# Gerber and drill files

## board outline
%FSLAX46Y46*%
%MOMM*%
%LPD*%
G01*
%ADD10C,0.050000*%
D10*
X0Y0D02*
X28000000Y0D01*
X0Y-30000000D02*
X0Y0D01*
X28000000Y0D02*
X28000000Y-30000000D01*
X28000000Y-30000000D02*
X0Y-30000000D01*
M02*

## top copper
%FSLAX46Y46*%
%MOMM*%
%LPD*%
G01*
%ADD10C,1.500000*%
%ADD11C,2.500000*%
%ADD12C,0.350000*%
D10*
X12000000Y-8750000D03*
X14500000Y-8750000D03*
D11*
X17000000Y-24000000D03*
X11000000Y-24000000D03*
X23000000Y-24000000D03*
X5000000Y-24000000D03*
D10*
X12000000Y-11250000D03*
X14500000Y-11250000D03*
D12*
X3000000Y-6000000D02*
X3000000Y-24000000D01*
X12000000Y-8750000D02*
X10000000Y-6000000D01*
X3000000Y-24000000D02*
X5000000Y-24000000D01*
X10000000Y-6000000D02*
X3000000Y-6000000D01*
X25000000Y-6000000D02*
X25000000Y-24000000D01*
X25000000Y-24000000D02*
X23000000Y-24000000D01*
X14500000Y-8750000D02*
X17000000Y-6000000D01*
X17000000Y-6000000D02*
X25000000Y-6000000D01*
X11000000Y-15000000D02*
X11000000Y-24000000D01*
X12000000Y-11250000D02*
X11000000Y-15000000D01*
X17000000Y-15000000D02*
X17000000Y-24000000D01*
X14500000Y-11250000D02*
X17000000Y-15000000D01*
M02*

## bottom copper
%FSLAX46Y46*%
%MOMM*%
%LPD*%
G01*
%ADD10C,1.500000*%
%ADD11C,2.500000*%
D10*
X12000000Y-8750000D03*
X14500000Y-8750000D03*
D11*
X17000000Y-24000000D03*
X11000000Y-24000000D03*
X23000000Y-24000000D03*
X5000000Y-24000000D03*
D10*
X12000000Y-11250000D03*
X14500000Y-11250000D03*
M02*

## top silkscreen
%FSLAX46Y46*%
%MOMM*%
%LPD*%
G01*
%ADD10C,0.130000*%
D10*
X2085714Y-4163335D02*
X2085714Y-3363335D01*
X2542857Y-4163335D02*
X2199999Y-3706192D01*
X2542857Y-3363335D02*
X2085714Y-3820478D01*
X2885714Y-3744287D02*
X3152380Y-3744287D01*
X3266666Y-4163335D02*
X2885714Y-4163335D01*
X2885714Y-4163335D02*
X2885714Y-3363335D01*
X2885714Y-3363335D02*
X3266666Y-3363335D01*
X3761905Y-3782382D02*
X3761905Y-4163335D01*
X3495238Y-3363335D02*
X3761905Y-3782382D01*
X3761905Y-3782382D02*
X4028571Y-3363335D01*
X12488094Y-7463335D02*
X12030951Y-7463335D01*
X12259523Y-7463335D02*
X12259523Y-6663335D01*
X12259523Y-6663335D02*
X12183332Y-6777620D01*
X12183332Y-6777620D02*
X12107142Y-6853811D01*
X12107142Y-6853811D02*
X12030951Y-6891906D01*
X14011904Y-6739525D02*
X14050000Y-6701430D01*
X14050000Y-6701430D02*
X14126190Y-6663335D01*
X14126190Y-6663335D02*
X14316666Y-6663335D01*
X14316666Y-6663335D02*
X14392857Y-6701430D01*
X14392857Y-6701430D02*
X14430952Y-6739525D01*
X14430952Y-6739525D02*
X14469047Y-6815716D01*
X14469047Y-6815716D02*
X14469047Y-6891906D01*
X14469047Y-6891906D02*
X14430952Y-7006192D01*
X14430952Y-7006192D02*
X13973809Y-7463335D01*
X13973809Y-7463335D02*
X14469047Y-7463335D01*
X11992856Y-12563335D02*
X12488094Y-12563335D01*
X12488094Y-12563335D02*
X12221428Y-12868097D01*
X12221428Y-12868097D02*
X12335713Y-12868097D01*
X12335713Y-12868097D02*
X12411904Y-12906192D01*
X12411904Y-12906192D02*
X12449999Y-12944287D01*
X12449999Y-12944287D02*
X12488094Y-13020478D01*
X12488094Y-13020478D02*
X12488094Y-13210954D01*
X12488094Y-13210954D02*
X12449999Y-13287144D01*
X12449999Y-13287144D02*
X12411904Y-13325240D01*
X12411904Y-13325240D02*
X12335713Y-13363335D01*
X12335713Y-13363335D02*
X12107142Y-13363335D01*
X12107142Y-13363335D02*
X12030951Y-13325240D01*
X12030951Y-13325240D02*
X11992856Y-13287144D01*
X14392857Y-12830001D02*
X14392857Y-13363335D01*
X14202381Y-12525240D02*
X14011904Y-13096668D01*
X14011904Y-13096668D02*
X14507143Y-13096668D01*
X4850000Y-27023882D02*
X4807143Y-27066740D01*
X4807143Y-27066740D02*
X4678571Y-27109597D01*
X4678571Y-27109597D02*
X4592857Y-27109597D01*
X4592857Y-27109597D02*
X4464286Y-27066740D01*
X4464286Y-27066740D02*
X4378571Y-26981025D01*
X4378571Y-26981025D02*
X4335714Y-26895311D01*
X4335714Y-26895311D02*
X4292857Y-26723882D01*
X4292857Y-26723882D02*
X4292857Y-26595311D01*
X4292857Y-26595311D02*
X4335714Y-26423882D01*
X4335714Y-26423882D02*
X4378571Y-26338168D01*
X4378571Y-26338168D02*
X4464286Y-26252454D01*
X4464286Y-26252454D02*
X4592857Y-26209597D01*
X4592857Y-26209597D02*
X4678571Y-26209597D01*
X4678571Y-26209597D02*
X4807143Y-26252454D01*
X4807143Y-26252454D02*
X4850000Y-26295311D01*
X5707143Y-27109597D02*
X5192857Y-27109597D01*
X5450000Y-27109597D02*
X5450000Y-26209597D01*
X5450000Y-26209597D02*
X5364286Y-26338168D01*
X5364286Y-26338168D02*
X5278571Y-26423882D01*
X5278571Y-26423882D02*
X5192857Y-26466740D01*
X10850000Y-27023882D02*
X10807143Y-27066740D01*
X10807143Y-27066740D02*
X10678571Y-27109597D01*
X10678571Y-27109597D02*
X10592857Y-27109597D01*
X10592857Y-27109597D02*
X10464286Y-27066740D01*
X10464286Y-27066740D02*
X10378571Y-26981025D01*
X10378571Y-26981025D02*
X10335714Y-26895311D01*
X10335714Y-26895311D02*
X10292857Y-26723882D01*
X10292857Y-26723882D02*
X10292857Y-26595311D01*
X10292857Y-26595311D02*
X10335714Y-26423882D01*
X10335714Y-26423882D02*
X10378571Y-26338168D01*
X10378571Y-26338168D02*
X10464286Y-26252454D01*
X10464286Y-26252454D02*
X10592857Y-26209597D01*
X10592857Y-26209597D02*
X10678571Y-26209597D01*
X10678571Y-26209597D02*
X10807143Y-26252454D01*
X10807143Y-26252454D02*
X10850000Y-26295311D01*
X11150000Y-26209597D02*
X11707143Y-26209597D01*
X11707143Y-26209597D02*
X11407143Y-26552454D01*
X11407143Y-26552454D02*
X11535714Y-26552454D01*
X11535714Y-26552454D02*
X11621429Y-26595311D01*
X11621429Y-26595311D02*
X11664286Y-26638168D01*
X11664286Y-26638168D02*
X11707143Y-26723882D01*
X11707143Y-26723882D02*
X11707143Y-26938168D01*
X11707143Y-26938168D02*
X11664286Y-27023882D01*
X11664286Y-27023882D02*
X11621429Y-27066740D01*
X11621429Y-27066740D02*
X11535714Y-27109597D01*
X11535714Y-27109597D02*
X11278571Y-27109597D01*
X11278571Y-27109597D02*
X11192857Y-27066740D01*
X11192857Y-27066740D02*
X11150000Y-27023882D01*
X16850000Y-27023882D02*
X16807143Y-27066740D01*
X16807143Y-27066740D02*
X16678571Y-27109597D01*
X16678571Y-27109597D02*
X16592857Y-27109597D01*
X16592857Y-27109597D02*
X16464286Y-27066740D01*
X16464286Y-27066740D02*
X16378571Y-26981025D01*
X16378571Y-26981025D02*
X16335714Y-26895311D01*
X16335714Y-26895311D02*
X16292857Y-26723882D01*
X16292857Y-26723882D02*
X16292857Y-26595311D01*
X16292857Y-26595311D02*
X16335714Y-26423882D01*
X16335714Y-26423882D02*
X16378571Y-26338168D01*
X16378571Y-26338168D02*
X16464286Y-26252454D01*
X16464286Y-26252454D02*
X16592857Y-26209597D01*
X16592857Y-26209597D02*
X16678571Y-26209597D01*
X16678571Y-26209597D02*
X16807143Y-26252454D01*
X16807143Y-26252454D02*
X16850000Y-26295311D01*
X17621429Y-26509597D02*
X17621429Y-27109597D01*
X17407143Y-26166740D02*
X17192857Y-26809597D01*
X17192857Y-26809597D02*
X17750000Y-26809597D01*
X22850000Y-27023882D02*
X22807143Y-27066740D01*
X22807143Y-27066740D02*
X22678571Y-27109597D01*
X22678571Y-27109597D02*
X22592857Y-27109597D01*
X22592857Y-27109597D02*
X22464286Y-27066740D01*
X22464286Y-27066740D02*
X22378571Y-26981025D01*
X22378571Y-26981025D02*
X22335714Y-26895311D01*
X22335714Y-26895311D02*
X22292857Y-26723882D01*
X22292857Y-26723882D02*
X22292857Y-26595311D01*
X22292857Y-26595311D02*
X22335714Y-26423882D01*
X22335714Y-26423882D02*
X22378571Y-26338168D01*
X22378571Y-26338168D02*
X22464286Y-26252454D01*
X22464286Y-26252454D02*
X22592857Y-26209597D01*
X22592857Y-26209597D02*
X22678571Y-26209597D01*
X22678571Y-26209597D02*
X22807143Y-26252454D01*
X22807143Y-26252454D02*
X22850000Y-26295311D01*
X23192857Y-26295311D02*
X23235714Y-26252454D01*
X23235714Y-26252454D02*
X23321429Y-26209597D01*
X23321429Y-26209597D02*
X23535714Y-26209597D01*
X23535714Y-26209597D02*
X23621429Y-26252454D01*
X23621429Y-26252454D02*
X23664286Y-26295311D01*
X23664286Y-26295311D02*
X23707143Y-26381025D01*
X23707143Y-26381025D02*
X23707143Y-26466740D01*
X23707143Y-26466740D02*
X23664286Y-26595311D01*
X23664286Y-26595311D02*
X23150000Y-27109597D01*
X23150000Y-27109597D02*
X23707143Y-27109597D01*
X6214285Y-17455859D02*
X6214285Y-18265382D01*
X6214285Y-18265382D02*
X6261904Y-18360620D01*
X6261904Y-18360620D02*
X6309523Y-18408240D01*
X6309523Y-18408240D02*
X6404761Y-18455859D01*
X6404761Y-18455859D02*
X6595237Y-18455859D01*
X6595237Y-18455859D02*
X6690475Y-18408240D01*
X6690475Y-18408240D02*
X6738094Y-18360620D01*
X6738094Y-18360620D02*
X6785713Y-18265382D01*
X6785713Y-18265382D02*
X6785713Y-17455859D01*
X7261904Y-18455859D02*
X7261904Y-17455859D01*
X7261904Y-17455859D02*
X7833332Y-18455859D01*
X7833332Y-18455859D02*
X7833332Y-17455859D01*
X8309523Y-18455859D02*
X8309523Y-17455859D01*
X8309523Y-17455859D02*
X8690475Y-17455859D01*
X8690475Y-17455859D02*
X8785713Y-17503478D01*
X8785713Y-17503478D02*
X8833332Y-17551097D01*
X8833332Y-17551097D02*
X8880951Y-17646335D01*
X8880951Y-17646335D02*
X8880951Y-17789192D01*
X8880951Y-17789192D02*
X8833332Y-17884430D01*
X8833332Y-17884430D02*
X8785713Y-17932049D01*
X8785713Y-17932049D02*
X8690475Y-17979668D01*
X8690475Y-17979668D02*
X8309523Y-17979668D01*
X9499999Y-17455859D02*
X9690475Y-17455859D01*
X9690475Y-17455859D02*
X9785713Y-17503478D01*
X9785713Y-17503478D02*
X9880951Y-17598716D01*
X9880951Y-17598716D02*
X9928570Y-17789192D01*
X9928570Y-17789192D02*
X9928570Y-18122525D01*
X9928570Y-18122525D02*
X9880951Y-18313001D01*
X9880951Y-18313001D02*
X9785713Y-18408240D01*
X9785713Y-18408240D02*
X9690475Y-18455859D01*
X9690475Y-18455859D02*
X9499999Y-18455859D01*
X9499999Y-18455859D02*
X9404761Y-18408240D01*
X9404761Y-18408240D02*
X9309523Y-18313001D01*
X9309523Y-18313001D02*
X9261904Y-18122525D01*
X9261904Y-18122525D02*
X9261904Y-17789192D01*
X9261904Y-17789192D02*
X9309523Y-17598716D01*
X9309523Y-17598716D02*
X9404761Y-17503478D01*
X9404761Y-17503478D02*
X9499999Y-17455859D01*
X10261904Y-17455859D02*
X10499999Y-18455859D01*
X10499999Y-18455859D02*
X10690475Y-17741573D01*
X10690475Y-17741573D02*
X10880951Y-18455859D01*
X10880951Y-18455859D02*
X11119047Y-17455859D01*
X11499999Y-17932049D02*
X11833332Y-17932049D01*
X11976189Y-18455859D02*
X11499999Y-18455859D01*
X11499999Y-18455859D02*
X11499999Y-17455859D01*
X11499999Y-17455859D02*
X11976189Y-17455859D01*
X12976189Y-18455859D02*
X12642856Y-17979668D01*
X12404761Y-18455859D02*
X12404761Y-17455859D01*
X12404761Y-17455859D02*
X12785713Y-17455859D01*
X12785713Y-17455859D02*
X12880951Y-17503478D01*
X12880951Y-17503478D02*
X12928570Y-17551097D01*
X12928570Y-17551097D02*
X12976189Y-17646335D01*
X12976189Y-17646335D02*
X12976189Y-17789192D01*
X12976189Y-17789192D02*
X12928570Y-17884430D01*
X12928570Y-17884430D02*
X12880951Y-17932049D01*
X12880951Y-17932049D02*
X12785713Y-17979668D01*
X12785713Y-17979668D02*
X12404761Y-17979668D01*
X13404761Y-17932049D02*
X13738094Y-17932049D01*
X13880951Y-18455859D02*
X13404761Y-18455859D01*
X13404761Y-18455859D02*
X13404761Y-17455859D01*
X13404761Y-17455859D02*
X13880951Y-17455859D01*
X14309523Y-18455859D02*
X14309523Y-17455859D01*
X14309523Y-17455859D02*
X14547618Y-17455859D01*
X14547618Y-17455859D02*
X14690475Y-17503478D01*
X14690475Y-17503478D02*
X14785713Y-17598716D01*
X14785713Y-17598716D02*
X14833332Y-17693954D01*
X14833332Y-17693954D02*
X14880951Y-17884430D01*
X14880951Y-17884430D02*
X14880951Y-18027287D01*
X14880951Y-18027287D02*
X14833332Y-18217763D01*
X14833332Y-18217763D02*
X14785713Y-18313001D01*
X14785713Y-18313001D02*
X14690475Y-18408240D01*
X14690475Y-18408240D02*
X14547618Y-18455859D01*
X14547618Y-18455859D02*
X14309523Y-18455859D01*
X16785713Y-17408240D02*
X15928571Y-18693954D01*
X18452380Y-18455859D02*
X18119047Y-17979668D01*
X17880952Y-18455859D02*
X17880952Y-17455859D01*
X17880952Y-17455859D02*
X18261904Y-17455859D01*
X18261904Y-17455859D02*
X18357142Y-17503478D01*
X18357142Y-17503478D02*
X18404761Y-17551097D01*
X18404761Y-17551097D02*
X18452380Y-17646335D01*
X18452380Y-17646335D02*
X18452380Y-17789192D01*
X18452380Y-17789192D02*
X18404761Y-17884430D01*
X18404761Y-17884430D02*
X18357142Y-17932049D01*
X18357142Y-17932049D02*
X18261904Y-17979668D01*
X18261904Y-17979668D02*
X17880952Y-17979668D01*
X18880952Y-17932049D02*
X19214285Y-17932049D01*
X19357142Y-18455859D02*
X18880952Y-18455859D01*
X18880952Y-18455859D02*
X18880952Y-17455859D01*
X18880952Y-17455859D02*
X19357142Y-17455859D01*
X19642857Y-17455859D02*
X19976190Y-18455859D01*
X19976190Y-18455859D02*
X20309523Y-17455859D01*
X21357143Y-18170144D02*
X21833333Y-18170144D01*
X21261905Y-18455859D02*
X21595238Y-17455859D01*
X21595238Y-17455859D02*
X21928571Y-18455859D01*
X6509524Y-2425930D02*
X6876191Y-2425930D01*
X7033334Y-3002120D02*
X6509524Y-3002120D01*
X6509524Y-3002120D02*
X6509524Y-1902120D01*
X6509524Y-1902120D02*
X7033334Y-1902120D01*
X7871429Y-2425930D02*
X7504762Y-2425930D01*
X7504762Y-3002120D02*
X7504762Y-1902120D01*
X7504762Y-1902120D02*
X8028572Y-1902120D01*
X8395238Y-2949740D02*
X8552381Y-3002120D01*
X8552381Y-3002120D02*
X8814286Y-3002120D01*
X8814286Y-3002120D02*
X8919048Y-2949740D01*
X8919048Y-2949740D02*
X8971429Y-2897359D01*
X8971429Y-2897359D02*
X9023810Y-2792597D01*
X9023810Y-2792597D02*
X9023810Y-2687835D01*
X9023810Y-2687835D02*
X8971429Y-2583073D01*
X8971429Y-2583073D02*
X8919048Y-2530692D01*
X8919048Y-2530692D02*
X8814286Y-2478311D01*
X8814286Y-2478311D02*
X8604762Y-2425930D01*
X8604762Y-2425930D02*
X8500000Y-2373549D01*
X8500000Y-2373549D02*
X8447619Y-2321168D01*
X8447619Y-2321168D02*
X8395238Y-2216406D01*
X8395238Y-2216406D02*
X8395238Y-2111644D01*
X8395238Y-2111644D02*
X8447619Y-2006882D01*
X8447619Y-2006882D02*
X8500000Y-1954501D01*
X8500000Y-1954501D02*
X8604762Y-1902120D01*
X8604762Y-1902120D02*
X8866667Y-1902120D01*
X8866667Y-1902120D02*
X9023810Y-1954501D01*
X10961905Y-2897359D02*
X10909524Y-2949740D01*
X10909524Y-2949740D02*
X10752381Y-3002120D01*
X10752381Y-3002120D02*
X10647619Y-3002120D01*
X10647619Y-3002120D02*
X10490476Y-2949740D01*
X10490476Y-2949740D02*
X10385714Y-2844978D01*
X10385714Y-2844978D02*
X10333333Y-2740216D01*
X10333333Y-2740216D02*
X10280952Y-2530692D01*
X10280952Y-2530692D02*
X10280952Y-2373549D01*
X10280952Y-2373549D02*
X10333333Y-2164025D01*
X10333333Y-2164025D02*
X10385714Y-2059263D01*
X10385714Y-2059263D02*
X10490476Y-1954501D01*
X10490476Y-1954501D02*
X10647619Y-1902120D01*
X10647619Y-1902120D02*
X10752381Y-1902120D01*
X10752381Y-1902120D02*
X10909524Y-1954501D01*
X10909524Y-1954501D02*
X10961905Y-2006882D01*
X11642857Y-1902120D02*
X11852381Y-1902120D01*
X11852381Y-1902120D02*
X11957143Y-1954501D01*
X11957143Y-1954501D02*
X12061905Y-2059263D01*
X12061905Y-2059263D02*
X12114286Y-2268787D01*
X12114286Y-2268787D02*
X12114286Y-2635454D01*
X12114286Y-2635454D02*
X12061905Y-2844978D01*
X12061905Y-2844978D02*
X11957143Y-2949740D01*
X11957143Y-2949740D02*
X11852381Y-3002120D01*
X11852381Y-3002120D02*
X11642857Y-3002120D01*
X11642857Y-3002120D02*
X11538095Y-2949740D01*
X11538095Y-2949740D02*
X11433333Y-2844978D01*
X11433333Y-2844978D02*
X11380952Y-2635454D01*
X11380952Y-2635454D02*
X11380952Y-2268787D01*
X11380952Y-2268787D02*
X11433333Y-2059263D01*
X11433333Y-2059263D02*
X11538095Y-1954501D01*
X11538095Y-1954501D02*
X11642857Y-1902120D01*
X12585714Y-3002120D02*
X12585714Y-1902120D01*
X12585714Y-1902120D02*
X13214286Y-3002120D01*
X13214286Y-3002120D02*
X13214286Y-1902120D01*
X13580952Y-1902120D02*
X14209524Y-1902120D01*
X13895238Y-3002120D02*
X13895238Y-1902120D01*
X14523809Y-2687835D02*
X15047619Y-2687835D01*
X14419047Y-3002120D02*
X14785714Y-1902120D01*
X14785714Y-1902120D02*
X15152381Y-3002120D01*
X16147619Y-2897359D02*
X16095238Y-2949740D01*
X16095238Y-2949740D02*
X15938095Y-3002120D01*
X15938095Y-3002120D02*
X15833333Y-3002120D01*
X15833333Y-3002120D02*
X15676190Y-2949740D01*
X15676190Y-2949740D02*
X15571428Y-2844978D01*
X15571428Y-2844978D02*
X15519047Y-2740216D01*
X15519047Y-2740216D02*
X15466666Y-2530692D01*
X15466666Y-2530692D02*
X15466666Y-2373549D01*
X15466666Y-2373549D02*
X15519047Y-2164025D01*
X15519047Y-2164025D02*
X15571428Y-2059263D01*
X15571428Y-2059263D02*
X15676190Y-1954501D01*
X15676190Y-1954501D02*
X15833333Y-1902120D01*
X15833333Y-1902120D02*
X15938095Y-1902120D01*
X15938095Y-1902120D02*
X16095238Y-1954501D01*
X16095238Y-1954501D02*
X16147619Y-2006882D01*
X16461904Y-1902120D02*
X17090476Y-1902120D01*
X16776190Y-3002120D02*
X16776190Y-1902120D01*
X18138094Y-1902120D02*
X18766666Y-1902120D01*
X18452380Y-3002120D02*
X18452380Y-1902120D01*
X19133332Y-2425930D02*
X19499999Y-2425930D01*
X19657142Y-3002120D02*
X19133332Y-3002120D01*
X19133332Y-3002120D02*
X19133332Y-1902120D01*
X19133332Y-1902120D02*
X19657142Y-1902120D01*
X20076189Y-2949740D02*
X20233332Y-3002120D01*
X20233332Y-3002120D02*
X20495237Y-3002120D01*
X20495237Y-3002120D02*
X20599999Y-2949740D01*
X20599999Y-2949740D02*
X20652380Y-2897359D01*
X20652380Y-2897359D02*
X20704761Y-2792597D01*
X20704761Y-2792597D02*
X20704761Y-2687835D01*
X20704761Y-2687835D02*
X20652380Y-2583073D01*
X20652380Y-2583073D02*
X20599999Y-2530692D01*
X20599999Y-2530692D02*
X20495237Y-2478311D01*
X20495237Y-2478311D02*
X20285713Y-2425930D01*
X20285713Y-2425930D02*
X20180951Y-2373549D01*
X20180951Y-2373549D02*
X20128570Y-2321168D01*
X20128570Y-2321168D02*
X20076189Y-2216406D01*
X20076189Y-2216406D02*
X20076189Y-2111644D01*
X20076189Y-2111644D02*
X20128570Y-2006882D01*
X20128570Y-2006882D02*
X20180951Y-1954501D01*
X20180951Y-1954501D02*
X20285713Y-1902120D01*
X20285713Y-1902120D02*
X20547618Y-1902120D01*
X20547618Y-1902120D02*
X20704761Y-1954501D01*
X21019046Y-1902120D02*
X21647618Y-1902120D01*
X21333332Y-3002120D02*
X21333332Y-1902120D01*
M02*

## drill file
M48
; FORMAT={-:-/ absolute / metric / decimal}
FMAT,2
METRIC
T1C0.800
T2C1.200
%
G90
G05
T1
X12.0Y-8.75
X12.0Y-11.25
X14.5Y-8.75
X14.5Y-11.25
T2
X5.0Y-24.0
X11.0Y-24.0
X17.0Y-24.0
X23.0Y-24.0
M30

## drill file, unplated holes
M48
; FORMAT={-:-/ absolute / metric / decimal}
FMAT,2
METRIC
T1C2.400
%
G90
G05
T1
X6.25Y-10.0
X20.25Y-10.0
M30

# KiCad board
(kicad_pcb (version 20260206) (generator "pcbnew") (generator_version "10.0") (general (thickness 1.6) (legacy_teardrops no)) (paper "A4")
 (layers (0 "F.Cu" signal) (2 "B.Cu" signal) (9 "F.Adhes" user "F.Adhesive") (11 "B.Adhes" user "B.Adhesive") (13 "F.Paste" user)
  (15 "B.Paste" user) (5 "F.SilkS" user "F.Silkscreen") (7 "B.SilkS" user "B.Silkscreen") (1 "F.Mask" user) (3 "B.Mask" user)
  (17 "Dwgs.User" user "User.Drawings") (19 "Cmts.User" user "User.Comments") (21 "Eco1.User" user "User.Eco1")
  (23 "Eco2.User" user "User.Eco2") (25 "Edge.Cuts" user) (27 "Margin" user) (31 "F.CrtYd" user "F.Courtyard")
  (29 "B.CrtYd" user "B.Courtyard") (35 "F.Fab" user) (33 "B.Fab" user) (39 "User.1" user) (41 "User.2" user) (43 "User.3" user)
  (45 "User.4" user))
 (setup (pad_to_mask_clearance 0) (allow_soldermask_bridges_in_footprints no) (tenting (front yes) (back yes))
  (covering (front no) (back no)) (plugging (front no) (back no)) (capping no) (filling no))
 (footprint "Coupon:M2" (layer "F.Cu") (at 6.25 10)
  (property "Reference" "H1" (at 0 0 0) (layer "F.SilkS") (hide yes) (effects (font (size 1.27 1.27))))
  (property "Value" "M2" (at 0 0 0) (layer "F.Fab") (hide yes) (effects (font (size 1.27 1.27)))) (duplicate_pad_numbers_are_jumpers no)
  (pad "" np_thru_hole circle (at 0 0) (size 2.4 2.4) (drill 2.4) (layers "*.Cu" "*.Mask")))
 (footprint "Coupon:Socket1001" (layer "F.Cu") (at 12 8.75)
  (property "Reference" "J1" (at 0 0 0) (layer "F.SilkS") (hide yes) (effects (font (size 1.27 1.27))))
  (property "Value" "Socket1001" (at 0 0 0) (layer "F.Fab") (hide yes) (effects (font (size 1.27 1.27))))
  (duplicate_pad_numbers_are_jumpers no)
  (pad "1" thru_hole circle (at 0 0) (size 1.5 1.5) (drill 0.8) (layers "*.Cu" "*.Mask") (remove_unused_layers no) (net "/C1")))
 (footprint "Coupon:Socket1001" (layer "F.Cu") (at 14.5 8.75)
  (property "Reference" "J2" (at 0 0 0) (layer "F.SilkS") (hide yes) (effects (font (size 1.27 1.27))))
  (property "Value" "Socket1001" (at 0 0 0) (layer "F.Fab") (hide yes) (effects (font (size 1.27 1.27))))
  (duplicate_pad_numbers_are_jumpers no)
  (pad "1" thru_hole circle (at 0 0) (size 1.5 1.5) (drill 0.8) (layers "*.Cu" "*.Mask") (remove_unused_layers no) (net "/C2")))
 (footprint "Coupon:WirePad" (layer "F.Cu") (at 17 24)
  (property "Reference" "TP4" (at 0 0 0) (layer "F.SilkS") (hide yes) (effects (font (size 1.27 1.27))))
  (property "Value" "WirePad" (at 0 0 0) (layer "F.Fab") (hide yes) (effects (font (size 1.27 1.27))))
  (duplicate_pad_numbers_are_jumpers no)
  (pad "1" thru_hole circle (at 0 0) (size 2.5 2.5) (drill 1.2) (layers "*.Cu" "*.Mask") (remove_unused_layers no) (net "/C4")))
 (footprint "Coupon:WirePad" (layer "F.Cu") (at 11 24)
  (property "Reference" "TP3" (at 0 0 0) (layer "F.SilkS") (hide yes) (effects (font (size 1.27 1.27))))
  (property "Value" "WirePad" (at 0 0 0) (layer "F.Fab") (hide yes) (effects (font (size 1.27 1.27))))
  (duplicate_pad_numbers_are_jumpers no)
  (pad "1" thru_hole circle (at 0 0) (size 2.5 2.5) (drill 1.2) (layers "*.Cu" "*.Mask") (remove_unused_layers no) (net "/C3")))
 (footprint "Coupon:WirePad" (layer "F.Cu") (at 23 24)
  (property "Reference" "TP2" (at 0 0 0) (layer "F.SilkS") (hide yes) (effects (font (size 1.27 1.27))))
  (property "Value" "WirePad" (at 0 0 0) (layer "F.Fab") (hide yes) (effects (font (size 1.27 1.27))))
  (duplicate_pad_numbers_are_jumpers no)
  (pad "1" thru_hole circle (at 0 0) (size 2.5 2.5) (drill 1.2) (layers "*.Cu" "*.Mask") (remove_unused_layers no) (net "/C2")))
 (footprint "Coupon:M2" (layer "F.Cu") (at 20.25 10)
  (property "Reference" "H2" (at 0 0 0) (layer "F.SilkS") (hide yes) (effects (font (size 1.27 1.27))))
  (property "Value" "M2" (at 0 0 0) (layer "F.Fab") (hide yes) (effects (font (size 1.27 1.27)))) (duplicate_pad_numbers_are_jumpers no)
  (pad "" np_thru_hole circle (at 0 0) (size 2.4 2.4) (drill 2.4) (layers "*.Cu" "*.Mask")))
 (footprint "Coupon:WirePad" (layer "F.Cu") (at 5 24)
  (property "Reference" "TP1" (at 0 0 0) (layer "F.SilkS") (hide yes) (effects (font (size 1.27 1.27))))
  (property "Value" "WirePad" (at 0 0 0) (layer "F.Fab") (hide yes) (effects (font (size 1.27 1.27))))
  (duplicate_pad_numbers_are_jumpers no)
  (pad "1" thru_hole circle (at 0 0) (size 2.5 2.5) (drill 1.2) (layers "*.Cu" "*.Mask") (remove_unused_layers no) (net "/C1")))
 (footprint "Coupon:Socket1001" (layer "F.Cu") (at 12 11.25)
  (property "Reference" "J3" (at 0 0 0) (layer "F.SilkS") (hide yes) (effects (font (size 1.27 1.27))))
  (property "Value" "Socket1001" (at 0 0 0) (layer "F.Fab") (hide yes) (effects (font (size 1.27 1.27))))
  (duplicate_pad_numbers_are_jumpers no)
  (pad "1" thru_hole circle (at 0 0) (size 1.5 1.5) (drill 0.8) (layers "*.Cu" "*.Mask") (remove_unused_layers no) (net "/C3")))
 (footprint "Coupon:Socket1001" (layer "F.Cu") (at 14.5 11.25)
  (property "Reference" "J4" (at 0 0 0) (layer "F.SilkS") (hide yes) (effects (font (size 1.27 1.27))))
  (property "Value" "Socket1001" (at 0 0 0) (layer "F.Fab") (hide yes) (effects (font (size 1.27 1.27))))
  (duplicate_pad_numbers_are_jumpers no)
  (pad "1" thru_hole circle (at 0 0) (size 1.5 1.5) (drill 0.8) (layers "*.Cu" "*.Mask") (remove_unused_layers no) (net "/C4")))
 (gr_line (start 0 0) (end 28 0) (stroke (width 0.05) (type default)) (layer "Edge.Cuts"))
 (gr_line (start 0 30) (end 0 0) (stroke (width 0.05) (type default)) (layer "Edge.Cuts"))
 (gr_line (start 28 0) (end 28 30) (stroke (width 0.05) (type default)) (layer "Edge.Cuts"))
 (gr_line (start 28 30) (end 0 30) (stroke (width 0.05) (type default)) (layer "Edge.Cuts"))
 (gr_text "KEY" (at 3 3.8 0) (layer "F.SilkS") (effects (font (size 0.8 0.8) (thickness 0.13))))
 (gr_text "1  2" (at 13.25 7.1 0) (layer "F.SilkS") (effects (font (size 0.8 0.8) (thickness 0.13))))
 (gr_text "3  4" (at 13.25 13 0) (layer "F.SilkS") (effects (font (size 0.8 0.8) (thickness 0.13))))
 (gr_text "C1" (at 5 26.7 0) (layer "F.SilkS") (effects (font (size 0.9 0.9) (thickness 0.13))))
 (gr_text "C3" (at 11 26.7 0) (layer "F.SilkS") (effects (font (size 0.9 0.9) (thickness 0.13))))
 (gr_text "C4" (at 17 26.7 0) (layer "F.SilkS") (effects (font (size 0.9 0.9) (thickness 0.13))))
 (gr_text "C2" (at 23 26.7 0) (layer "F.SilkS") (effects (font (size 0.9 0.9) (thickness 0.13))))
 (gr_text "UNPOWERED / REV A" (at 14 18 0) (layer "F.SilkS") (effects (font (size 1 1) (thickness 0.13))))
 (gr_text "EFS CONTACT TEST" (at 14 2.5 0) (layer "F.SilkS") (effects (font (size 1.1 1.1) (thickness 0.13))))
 (segment (start 3 6) (end 3 24) (width 0.35) (layer "F.Cu") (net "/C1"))
 (segment (start 12 8.75) (end 10 6) (width 0.35) (layer "F.Cu") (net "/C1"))
 (segment (start 3 24) (end 5 24) (width 0.35) (layer "F.Cu") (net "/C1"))
 (segment (start 10 6) (end 3 6) (width 0.35) (layer "F.Cu") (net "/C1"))
 (segment (start 25 6) (end 25 24) (width 0.35) (layer "F.Cu") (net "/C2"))
 (segment (start 25 24) (end 23 24) (width 0.35) (layer "F.Cu") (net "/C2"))
 (segment (start 14.5 8.75) (end 17 6) (width 0.35) (layer "F.Cu") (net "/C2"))
 (segment (start 17 6) (end 25 6) (width 0.35) (layer "F.Cu") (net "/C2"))
 (segment (start 11 15) (end 11 24) (width 0.35) (layer "F.Cu") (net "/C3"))
 (segment (start 12 11.25) (end 11 15) (width 0.35) (layer "F.Cu") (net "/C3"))
 (segment (start 17 15) (end 17 24) (width 0.35) (layer "F.Cu") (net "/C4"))
 (segment (start 14.5 11.25) (end 17 15) (width 0.35) (layer "F.Cu") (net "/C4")))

